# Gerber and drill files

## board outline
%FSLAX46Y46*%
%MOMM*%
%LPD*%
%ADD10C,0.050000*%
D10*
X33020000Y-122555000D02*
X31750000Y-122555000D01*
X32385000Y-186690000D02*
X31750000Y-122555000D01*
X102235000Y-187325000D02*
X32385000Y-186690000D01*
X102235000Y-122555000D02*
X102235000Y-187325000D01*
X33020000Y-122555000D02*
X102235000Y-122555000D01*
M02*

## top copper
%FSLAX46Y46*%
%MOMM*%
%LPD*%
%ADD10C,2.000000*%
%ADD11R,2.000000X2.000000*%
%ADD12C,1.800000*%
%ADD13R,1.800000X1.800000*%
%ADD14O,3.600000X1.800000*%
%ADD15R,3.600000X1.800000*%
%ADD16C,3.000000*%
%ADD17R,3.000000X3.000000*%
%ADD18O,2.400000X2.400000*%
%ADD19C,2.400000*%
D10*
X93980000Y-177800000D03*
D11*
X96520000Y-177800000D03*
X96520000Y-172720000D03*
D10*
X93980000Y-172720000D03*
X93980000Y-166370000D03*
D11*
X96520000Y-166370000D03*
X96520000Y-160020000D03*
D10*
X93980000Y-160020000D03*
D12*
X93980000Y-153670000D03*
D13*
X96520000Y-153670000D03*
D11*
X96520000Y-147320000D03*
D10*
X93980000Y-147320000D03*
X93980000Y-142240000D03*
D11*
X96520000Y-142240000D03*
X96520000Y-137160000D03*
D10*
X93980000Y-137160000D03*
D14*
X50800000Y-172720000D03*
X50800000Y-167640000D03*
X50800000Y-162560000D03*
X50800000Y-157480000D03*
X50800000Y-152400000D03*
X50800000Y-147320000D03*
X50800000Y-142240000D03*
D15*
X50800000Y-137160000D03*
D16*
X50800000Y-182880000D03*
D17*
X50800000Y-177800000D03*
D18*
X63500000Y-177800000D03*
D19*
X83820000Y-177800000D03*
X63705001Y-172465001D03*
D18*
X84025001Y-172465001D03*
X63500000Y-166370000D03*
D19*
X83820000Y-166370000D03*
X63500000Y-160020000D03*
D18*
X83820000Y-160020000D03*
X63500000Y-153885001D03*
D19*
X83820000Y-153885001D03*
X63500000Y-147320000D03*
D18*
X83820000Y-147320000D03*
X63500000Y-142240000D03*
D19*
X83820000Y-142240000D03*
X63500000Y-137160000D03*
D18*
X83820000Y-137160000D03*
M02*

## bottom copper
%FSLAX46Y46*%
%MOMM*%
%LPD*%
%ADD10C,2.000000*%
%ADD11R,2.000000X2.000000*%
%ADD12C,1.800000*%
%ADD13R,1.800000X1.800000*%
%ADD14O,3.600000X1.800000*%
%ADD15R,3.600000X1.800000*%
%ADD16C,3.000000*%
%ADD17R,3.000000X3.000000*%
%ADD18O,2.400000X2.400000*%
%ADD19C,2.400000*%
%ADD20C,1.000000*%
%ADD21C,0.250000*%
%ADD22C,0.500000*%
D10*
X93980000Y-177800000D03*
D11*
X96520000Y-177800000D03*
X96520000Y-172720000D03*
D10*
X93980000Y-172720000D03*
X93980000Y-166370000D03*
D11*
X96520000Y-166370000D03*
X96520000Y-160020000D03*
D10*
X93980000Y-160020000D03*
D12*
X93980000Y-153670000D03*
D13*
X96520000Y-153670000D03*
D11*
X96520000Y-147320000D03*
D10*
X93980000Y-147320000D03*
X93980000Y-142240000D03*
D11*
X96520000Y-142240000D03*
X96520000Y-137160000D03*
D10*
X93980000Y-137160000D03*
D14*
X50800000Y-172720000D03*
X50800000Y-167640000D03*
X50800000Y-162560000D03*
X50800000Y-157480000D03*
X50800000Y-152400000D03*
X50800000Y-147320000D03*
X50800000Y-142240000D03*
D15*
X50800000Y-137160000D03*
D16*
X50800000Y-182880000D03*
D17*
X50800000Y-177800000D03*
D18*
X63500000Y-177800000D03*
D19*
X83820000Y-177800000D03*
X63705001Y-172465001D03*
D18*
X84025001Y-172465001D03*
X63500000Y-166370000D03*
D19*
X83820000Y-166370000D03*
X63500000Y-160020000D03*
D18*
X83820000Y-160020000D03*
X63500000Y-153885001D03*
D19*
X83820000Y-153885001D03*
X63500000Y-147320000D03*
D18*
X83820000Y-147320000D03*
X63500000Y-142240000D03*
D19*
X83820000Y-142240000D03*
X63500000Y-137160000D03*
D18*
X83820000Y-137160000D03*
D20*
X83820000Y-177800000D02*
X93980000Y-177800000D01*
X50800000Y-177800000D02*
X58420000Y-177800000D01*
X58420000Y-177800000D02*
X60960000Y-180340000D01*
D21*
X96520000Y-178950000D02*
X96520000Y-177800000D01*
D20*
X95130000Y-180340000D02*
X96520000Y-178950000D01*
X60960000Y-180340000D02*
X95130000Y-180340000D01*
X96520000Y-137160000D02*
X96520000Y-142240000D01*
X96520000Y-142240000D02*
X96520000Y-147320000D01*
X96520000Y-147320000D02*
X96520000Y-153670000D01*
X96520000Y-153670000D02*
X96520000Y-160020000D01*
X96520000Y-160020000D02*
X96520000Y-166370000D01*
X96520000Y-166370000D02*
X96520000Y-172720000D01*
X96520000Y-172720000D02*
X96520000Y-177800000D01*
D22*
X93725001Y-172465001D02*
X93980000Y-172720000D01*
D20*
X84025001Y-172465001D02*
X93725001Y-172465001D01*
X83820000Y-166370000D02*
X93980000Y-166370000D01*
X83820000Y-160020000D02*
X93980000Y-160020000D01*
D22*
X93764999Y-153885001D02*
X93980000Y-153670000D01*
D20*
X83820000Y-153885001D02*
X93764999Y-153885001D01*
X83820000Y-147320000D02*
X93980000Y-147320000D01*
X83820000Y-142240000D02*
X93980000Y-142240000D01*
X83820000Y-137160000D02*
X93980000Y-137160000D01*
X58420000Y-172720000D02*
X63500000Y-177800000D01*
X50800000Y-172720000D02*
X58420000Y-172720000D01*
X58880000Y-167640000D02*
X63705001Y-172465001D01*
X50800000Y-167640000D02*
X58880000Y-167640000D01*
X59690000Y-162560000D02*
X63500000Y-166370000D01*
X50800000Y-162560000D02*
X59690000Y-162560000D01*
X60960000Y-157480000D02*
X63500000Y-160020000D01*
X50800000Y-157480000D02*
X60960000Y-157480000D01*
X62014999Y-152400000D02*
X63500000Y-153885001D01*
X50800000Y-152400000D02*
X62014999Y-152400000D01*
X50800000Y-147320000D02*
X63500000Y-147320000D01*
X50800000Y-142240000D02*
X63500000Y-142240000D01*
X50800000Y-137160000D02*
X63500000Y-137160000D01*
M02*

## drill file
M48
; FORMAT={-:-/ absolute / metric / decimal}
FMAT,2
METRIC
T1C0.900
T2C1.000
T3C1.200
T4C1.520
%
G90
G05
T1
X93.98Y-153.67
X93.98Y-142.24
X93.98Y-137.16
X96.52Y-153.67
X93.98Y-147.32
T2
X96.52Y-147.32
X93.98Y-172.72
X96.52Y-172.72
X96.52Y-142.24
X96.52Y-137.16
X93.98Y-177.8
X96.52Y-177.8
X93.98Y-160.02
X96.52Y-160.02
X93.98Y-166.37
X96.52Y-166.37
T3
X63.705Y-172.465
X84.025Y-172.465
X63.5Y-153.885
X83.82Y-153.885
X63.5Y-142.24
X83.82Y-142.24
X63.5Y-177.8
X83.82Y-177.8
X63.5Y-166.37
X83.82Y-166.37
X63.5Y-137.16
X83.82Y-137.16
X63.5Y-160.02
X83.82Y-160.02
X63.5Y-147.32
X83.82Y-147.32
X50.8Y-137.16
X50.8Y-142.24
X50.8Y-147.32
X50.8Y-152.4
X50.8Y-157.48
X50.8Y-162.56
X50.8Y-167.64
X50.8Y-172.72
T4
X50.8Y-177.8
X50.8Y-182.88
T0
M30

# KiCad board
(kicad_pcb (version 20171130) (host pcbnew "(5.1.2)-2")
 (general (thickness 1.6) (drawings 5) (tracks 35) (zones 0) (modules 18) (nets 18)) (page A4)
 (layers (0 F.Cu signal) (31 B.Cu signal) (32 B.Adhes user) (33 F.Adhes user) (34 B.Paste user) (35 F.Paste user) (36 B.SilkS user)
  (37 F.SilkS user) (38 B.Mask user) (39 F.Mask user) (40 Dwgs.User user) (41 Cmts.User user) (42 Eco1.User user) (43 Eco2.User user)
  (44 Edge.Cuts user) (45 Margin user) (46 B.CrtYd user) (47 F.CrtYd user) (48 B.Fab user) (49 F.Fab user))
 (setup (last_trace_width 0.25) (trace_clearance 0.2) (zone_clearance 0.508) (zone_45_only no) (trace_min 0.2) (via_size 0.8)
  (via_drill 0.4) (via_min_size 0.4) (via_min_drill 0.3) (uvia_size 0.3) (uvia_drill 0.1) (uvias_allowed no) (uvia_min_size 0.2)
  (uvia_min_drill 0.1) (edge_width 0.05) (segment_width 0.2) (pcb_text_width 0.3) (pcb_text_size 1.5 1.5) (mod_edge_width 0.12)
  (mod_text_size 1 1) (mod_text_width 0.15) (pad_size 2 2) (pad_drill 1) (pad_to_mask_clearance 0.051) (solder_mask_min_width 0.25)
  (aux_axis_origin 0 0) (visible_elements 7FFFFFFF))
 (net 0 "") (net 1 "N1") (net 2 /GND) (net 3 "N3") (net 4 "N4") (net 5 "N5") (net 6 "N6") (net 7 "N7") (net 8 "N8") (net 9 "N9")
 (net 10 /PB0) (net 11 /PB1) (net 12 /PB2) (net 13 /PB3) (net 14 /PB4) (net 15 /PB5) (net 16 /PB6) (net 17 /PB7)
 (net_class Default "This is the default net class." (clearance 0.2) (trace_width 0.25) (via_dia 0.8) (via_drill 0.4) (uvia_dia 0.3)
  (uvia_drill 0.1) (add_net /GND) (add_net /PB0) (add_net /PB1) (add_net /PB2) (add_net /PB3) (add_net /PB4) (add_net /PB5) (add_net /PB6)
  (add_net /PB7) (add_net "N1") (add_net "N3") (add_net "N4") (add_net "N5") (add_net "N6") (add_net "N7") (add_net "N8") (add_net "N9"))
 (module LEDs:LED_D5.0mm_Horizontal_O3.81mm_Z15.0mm (layer F.Cu) (at 96.52 177.8 180)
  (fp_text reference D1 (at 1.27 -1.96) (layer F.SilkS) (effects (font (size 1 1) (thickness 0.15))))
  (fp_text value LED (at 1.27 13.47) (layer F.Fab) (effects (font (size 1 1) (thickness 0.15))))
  (pad 2 thru_hole circle (at 2.54 0 180) (size 2 2) (drill 1) (layers *.Cu *.Mask) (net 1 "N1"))
  (pad 1 thru_hole rect (at 0 0 180) (size 2 2) (drill 1) (layers *.Cu *.Mask) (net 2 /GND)))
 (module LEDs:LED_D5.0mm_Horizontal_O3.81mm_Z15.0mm (layer F.Cu) (at 96.52 172.72 180)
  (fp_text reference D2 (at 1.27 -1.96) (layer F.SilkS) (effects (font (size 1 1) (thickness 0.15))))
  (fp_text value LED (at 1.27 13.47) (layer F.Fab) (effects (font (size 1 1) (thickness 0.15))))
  (pad 1 thru_hole rect (at 0 0 180) (size 2 2) (drill 1) (layers *.Cu *.Mask) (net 2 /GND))
  (pad 2 thru_hole circle (at 2.54 0 180) (size 2 2) (drill 1) (layers *.Cu *.Mask) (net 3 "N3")))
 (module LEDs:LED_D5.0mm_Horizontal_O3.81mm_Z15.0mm (layer F.Cu) (at 96.52 166.37 180)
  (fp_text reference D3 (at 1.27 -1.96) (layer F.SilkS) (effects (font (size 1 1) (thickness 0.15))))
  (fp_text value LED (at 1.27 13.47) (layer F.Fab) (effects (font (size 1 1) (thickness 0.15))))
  (pad 2 thru_hole circle (at 2.54 0 180) (size 2 2) (drill 1) (layers *.Cu *.Mask) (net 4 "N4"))
  (pad 1 thru_hole rect (at 0 0 180) (size 2 2) (drill 1) (layers *.Cu *.Mask) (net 2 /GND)))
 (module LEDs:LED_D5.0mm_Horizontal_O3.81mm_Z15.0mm (layer F.Cu) (at 96.52 160.02 180)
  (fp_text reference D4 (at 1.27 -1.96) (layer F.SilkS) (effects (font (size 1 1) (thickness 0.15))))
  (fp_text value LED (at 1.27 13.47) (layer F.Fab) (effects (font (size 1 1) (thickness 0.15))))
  (pad 1 thru_hole rect (at 0 0 180) (size 2 2) (drill 1) (layers *.Cu *.Mask) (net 2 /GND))
  (pad 2 thru_hole circle (at 2.54 0 180) (size 2 2) (drill 1) (layers *.Cu *.Mask) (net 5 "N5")))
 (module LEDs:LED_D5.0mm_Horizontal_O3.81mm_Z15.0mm (layer F.Cu) (at 96.52 153.67 180)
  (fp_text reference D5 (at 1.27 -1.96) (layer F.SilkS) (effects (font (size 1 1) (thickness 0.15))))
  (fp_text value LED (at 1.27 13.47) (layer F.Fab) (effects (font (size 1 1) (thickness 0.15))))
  (pad 2 thru_hole circle (at 2.54 0 180) (size 1.8 1.8) (drill 0.9) (layers *.Cu *.Mask) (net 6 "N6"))
  (pad 1 thru_hole rect (at 0 0 180) (size 1.8 1.8) (drill 0.9) (layers *.Cu *.Mask) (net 2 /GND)))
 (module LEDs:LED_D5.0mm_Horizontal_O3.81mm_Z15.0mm (layer F.Cu) (at 96.52 147.32 180)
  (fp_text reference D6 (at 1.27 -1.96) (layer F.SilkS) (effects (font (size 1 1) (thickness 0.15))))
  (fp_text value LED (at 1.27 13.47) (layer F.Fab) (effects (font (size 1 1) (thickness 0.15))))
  (pad 1 thru_hole rect (at 0 0 180) (size 2 2) (drill 1) (layers *.Cu *.Mask) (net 2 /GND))
  (pad 2 thru_hole circle (at 2.54 0 180) (size 2 2) (drill 0.9) (layers *.Cu *.Mask) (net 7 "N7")))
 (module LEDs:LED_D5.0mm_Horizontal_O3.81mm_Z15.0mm (layer F.Cu) (at 96.52 142.24 180)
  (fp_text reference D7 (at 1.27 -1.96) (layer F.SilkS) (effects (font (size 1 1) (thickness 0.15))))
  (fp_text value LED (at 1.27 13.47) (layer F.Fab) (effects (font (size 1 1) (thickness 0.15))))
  (pad 2 thru_hole circle (at 2.54 0 180) (size 2 2) (drill 0.9) (layers *.Cu *.Mask) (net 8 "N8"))
  (pad 1 thru_hole rect (at 0 0 180) (size 2 2) (drill 1) (layers *.Cu *.Mask) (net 2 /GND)))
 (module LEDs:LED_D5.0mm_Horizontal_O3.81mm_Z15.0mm (layer F.Cu) (at 96.52 137.16 180)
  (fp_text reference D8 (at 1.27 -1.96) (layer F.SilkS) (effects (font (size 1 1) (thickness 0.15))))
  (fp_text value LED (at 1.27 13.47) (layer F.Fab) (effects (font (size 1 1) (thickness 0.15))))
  (pad 1 thru_hole rect (at 0 0 180) (size 2 2) (drill 1) (layers *.Cu *.Mask) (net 2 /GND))
  (pad 2 thru_hole circle (at 2.54 0 180) (size 2 2) (drill 0.9) (layers *.Cu *.Mask) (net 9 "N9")))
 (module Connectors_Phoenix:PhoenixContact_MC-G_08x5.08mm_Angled (layer F.Cu) (at 50.8 137.16 270)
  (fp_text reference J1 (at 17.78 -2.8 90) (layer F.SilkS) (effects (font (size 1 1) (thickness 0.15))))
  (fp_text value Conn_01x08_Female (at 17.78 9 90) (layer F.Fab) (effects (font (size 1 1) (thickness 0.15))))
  (pad 8 thru_hole oval (at 35.56 0 270) (size 1.8 3.6) (drill 1.2) (layers *.Cu *.Mask) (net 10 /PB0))
  (pad 7 thru_hole oval (at 30.48 0 270) (size 1.8 3.6) (drill 1.2) (layers *.Cu *.Mask) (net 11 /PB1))
  (pad 6 thru_hole oval (at 25.4 0 270) (size 1.8 3.6) (drill 1.2) (layers *.Cu *.Mask) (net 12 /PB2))
  (pad 5 thru_hole oval (at 20.32 0 270) (size 1.8 3.6) (drill 1.2) (layers *.Cu *.Mask) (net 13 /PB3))
  (pad 4 thru_hole oval (at 15.24 0 270) (size 1.8 3.6) (drill 1.2) (layers *.Cu *.Mask) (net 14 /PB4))
  (pad 3 thru_hole oval (at 10.16 0 270) (size 1.8 3.6) (drill 1.2) (layers *.Cu *.Mask) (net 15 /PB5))
  (pad 2 thru_hole oval (at 5.08 0 270) (size 1.8 3.6) (drill 1.2) (layers *.Cu *.Mask) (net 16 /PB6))
  (pad 1 thru_hole rect (at 0 0 270) (size 1.8 3.6) (drill 1.2) (layers *.Cu *.Mask) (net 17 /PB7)))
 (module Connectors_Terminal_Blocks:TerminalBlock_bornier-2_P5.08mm (layer F.Cu) (at 50.8 177.8 270)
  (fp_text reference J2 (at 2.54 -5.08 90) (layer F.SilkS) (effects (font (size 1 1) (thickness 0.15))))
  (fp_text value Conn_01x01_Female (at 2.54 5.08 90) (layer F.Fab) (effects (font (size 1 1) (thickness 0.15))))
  (pad 2 thru_hole circle (at 5.08 0 270) (size 3 3) (drill 1.52) (layers *.Cu *.Mask))
  (pad 1 thru_hole rect (at 0 0 270) (size 3 3) (drill 1.52) (layers *.Cu *.Mask) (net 2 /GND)))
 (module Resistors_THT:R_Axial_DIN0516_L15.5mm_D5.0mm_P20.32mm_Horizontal (layer F.Cu) (at 83.82 177.8 180)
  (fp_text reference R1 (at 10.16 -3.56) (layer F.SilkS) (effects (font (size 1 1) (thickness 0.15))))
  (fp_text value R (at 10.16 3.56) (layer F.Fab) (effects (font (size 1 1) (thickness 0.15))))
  (pad 2 thru_hole oval (at 20.32 0 180) (size 2.4 2.4) (drill 1.2) (layers *.Cu *.Mask) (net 10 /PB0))
  (pad 1 thru_hole circle (at 0 0 180) (size 2.4 2.4) (drill 1.2) (layers *.Cu *.Mask) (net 1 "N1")))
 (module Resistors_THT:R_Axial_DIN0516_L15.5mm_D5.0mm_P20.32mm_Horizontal (layer F.Cu) (at 63.705001 172.465001)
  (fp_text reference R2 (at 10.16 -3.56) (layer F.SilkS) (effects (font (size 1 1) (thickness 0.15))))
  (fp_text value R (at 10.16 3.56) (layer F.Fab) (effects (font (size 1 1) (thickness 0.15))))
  (pad 1 thru_hole circle (at 0 0) (size 2.4 2.4) (drill 1.2) (layers *.Cu *.Mask) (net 11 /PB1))
  (pad 2 thru_hole oval (at 20.32 0) (size 2.4 2.4) (drill 1.2) (layers *.Cu *.Mask) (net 3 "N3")))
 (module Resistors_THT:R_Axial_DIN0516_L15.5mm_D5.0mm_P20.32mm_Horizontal (layer F.Cu) (at 83.82 166.37 180)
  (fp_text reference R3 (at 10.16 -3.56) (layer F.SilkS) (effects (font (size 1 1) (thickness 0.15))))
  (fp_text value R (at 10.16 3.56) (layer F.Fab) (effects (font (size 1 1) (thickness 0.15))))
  (pad 2 thru_hole oval (at 20.32 0 180) (size 2.4 2.4) (drill 1.2) (layers *.Cu *.Mask) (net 12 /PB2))
  (pad 1 thru_hole circle (at 0 0 180) (size 2.4 2.4) (drill 1.2) (layers *.Cu *.Mask) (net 4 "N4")))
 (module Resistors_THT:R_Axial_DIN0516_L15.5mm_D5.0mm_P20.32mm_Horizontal (layer F.Cu) (at 63.5 160.02)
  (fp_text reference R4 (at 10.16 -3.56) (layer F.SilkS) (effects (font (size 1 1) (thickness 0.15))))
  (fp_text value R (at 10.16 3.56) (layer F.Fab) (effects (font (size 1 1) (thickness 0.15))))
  (pad 1 thru_hole circle (at 0 0) (size 2.4 2.4) (drill 1.2) (layers *.Cu *.Mask) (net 13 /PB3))
  (pad 2 thru_hole oval (at 20.32 0) (size 2.4 2.4) (drill 1.2) (layers *.Cu *.Mask) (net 5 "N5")))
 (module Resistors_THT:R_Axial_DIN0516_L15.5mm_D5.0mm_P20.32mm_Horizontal (layer F.Cu) (at 83.82 153.885001 180)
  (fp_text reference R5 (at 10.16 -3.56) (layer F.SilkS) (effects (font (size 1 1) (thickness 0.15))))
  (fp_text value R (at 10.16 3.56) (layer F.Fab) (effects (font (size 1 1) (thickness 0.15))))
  (pad 2 thru_hole oval (at 20.32 0 180) (size 2.4 2.4) (drill 1.2) (layers *.Cu *.Mask) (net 14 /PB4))
  (pad 1 thru_hole circle (at 0 0 180) (size 2.4 2.4) (drill 1.2) (layers *.Cu *.Mask) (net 6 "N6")))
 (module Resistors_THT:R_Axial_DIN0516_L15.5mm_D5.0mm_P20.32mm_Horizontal (layer F.Cu) (at 63.5 147.32)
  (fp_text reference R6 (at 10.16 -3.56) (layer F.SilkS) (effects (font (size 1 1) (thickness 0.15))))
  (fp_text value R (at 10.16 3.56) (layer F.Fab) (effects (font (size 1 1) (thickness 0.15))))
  (pad 1 thru_hole circle (at 0 0) (size 2.4 2.4) (drill 1.2) (layers *.Cu *.Mask) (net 15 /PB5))
  (pad 2 thru_hole oval (at 20.32 0) (size 2.4 2.4) (drill 1.2) (layers *.Cu *.Mask) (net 7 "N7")))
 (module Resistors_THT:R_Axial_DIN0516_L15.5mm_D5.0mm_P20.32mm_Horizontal (layer F.Cu) (at 83.82 142.24 180)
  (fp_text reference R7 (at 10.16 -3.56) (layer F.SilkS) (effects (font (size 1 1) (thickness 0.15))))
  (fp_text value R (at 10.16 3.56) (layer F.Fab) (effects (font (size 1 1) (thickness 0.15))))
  (pad 2 thru_hole oval (at 20.32 0 180) (size 2.4 2.4) (drill 1.2) (layers *.Cu *.Mask) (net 16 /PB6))
  (pad 1 thru_hole circle (at 0 0 180) (size 2.4 2.4) (drill 1.2) (layers *.Cu *.Mask) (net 8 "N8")))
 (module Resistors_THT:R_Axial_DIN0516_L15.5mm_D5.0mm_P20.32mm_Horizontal (layer F.Cu) (at 63.5 137.16)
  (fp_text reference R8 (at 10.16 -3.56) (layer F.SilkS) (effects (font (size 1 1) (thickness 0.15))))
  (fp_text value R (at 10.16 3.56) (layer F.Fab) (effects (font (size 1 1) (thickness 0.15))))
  (pad 1 thru_hole circle (at 0 0) (size 2.4 2.4) (drill 1.2) (layers *.Cu *.Mask) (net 17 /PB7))
  (pad 2 thru_hole oval (at 20.32 0) (size 2.4 2.4) (drill 1.2) (layers *.Cu *.Mask) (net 9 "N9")))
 (gr_line (start 33.02 122.555) (end 31.75 122.555) (layer Edge.Cuts) (width 0.05))
 (gr_line (start 32.385 186.69) (end 31.75 122.555) (layer Edge.Cuts) (width 0.05))
 (gr_line (start 102.235 187.325) (end 32.385 186.69) (layer Edge.Cuts) (width 0.05))
 (gr_line (start 102.235 122.555) (end 102.235 187.325) (layer Edge.Cuts) (width 0.05))
 (gr_line (start 33.02 122.555) (end 102.235 122.555) (layer Edge.Cuts) (width 0.05))
 (segment (start 83.82 177.8) (end 93.98 177.8) (width 1) (layer B.Cu) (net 1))
 (segment (start 50.8 177.8) (end 58.42 177.8) (width 1) (layer B.Cu) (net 2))
 (segment (start 58.42 177.8) (end 60.96 180.34) (width 1) (layer B.Cu) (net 2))
 (segment (start 96.52 178.95) (end 96.52 177.8) (width 0.25) (layer B.Cu) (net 2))
 (segment (start 95.13 180.34) (end 96.52 178.95) (width 1) (layer B.Cu) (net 2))
 (segment (start 60.96 180.34) (end 95.13 180.34) (width 1) (layer B.Cu) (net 2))
 (segment (start 96.52 137.16) (end 96.52 142.24) (width 1) (layer B.Cu) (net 2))
 (segment (start 96.52 142.24) (end 96.52 147.32) (width 1) (layer B.Cu) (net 2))
 (segment (start 96.52 147.32) (end 96.52 153.67) (width 1) (layer B.Cu) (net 2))
 (segment (start 96.52 153.67) (end 96.52 160.02) (width 1) (layer B.Cu) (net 2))
 (segment (start 96.52 160.02) (end 96.52 166.37) (width 1) (layer B.Cu) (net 2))
 (segment (start 96.52 166.37) (end 96.52 172.72) (width 1) (layer B.Cu) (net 2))
 (segment (start 96.52 172.72) (end 96.52 177.8) (width 1) (layer B.Cu) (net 2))
 (segment (start 93.725001 172.465001) (end 93.98 172.72) (width 0.5) (layer B.Cu) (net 3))
 (segment (start 84.025001 172.465001) (end 93.725001 172.465001) (width 1) (layer B.Cu) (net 3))
 (segment (start 83.82 166.37) (end 93.98 166.37) (width 1) (layer B.Cu) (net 4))
 (segment (start 83.82 160.02) (end 93.98 160.02) (width 1) (layer B.Cu) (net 5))
 (segment (start 93.764999 153.885001) (end 93.98 153.67) (width 0.5) (layer B.Cu) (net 6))
 (segment (start 83.82 153.885001) (end 93.764999 153.885001) (width 1) (layer B.Cu) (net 6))
 (segment (start 83.82 147.32) (end 93.98 147.32) (width 1) (layer B.Cu) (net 7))
 (segment (start 83.82 142.24) (end 93.98 142.24) (width 1) (layer B.Cu) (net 8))
 (segment (start 83.82 137.16) (end 93.98 137.16) (width 1) (layer B.Cu) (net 9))
 (segment (start 58.42 172.72) (end 63.5 177.8) (width 1) (layer B.Cu) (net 10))
 (segment (start 50.8 172.72) (end 58.42 172.72) (width 1) (layer B.Cu) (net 10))
 (segment (start 58.88 167.64) (end 63.705001 172.465001) (width 1) (layer B.Cu) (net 11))
 (segment (start 50.8 167.64) (end 58.88 167.64) (width 1) (layer B.Cu) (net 11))
 (segment (start 59.69 162.56) (end 63.5 166.37) (width 1) (layer B.Cu) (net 12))
 (segment (start 50.8 162.56) (end 59.69 162.56) (width 1) (layer B.Cu) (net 12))
 (segment (start 60.96 157.48) (end 63.5 160.02) (width 1) (layer B.Cu) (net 13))
 (segment (start 50.8 157.48) (end 60.96 157.48) (width 1) (layer B.Cu) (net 13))
 (segment (start 62.014999 152.4) (end 63.5 153.885001) (width 1) (layer B.Cu) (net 14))
 (segment (start 50.8 152.4) (end 62.014999 152.4) (width 1) (layer B.Cu) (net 14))
 (segment (start 50.8 147.32) (end 63.5 147.32) (width 1) (layer B.Cu) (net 15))
 (segment (start 50.8 142.24) (end 63.5 142.24) (width 1) (layer B.Cu) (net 16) (status 40000))
 (segment (start 50.8 137.16) (end 63.5 137.16) (width 1) (layer B.Cu) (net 17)))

